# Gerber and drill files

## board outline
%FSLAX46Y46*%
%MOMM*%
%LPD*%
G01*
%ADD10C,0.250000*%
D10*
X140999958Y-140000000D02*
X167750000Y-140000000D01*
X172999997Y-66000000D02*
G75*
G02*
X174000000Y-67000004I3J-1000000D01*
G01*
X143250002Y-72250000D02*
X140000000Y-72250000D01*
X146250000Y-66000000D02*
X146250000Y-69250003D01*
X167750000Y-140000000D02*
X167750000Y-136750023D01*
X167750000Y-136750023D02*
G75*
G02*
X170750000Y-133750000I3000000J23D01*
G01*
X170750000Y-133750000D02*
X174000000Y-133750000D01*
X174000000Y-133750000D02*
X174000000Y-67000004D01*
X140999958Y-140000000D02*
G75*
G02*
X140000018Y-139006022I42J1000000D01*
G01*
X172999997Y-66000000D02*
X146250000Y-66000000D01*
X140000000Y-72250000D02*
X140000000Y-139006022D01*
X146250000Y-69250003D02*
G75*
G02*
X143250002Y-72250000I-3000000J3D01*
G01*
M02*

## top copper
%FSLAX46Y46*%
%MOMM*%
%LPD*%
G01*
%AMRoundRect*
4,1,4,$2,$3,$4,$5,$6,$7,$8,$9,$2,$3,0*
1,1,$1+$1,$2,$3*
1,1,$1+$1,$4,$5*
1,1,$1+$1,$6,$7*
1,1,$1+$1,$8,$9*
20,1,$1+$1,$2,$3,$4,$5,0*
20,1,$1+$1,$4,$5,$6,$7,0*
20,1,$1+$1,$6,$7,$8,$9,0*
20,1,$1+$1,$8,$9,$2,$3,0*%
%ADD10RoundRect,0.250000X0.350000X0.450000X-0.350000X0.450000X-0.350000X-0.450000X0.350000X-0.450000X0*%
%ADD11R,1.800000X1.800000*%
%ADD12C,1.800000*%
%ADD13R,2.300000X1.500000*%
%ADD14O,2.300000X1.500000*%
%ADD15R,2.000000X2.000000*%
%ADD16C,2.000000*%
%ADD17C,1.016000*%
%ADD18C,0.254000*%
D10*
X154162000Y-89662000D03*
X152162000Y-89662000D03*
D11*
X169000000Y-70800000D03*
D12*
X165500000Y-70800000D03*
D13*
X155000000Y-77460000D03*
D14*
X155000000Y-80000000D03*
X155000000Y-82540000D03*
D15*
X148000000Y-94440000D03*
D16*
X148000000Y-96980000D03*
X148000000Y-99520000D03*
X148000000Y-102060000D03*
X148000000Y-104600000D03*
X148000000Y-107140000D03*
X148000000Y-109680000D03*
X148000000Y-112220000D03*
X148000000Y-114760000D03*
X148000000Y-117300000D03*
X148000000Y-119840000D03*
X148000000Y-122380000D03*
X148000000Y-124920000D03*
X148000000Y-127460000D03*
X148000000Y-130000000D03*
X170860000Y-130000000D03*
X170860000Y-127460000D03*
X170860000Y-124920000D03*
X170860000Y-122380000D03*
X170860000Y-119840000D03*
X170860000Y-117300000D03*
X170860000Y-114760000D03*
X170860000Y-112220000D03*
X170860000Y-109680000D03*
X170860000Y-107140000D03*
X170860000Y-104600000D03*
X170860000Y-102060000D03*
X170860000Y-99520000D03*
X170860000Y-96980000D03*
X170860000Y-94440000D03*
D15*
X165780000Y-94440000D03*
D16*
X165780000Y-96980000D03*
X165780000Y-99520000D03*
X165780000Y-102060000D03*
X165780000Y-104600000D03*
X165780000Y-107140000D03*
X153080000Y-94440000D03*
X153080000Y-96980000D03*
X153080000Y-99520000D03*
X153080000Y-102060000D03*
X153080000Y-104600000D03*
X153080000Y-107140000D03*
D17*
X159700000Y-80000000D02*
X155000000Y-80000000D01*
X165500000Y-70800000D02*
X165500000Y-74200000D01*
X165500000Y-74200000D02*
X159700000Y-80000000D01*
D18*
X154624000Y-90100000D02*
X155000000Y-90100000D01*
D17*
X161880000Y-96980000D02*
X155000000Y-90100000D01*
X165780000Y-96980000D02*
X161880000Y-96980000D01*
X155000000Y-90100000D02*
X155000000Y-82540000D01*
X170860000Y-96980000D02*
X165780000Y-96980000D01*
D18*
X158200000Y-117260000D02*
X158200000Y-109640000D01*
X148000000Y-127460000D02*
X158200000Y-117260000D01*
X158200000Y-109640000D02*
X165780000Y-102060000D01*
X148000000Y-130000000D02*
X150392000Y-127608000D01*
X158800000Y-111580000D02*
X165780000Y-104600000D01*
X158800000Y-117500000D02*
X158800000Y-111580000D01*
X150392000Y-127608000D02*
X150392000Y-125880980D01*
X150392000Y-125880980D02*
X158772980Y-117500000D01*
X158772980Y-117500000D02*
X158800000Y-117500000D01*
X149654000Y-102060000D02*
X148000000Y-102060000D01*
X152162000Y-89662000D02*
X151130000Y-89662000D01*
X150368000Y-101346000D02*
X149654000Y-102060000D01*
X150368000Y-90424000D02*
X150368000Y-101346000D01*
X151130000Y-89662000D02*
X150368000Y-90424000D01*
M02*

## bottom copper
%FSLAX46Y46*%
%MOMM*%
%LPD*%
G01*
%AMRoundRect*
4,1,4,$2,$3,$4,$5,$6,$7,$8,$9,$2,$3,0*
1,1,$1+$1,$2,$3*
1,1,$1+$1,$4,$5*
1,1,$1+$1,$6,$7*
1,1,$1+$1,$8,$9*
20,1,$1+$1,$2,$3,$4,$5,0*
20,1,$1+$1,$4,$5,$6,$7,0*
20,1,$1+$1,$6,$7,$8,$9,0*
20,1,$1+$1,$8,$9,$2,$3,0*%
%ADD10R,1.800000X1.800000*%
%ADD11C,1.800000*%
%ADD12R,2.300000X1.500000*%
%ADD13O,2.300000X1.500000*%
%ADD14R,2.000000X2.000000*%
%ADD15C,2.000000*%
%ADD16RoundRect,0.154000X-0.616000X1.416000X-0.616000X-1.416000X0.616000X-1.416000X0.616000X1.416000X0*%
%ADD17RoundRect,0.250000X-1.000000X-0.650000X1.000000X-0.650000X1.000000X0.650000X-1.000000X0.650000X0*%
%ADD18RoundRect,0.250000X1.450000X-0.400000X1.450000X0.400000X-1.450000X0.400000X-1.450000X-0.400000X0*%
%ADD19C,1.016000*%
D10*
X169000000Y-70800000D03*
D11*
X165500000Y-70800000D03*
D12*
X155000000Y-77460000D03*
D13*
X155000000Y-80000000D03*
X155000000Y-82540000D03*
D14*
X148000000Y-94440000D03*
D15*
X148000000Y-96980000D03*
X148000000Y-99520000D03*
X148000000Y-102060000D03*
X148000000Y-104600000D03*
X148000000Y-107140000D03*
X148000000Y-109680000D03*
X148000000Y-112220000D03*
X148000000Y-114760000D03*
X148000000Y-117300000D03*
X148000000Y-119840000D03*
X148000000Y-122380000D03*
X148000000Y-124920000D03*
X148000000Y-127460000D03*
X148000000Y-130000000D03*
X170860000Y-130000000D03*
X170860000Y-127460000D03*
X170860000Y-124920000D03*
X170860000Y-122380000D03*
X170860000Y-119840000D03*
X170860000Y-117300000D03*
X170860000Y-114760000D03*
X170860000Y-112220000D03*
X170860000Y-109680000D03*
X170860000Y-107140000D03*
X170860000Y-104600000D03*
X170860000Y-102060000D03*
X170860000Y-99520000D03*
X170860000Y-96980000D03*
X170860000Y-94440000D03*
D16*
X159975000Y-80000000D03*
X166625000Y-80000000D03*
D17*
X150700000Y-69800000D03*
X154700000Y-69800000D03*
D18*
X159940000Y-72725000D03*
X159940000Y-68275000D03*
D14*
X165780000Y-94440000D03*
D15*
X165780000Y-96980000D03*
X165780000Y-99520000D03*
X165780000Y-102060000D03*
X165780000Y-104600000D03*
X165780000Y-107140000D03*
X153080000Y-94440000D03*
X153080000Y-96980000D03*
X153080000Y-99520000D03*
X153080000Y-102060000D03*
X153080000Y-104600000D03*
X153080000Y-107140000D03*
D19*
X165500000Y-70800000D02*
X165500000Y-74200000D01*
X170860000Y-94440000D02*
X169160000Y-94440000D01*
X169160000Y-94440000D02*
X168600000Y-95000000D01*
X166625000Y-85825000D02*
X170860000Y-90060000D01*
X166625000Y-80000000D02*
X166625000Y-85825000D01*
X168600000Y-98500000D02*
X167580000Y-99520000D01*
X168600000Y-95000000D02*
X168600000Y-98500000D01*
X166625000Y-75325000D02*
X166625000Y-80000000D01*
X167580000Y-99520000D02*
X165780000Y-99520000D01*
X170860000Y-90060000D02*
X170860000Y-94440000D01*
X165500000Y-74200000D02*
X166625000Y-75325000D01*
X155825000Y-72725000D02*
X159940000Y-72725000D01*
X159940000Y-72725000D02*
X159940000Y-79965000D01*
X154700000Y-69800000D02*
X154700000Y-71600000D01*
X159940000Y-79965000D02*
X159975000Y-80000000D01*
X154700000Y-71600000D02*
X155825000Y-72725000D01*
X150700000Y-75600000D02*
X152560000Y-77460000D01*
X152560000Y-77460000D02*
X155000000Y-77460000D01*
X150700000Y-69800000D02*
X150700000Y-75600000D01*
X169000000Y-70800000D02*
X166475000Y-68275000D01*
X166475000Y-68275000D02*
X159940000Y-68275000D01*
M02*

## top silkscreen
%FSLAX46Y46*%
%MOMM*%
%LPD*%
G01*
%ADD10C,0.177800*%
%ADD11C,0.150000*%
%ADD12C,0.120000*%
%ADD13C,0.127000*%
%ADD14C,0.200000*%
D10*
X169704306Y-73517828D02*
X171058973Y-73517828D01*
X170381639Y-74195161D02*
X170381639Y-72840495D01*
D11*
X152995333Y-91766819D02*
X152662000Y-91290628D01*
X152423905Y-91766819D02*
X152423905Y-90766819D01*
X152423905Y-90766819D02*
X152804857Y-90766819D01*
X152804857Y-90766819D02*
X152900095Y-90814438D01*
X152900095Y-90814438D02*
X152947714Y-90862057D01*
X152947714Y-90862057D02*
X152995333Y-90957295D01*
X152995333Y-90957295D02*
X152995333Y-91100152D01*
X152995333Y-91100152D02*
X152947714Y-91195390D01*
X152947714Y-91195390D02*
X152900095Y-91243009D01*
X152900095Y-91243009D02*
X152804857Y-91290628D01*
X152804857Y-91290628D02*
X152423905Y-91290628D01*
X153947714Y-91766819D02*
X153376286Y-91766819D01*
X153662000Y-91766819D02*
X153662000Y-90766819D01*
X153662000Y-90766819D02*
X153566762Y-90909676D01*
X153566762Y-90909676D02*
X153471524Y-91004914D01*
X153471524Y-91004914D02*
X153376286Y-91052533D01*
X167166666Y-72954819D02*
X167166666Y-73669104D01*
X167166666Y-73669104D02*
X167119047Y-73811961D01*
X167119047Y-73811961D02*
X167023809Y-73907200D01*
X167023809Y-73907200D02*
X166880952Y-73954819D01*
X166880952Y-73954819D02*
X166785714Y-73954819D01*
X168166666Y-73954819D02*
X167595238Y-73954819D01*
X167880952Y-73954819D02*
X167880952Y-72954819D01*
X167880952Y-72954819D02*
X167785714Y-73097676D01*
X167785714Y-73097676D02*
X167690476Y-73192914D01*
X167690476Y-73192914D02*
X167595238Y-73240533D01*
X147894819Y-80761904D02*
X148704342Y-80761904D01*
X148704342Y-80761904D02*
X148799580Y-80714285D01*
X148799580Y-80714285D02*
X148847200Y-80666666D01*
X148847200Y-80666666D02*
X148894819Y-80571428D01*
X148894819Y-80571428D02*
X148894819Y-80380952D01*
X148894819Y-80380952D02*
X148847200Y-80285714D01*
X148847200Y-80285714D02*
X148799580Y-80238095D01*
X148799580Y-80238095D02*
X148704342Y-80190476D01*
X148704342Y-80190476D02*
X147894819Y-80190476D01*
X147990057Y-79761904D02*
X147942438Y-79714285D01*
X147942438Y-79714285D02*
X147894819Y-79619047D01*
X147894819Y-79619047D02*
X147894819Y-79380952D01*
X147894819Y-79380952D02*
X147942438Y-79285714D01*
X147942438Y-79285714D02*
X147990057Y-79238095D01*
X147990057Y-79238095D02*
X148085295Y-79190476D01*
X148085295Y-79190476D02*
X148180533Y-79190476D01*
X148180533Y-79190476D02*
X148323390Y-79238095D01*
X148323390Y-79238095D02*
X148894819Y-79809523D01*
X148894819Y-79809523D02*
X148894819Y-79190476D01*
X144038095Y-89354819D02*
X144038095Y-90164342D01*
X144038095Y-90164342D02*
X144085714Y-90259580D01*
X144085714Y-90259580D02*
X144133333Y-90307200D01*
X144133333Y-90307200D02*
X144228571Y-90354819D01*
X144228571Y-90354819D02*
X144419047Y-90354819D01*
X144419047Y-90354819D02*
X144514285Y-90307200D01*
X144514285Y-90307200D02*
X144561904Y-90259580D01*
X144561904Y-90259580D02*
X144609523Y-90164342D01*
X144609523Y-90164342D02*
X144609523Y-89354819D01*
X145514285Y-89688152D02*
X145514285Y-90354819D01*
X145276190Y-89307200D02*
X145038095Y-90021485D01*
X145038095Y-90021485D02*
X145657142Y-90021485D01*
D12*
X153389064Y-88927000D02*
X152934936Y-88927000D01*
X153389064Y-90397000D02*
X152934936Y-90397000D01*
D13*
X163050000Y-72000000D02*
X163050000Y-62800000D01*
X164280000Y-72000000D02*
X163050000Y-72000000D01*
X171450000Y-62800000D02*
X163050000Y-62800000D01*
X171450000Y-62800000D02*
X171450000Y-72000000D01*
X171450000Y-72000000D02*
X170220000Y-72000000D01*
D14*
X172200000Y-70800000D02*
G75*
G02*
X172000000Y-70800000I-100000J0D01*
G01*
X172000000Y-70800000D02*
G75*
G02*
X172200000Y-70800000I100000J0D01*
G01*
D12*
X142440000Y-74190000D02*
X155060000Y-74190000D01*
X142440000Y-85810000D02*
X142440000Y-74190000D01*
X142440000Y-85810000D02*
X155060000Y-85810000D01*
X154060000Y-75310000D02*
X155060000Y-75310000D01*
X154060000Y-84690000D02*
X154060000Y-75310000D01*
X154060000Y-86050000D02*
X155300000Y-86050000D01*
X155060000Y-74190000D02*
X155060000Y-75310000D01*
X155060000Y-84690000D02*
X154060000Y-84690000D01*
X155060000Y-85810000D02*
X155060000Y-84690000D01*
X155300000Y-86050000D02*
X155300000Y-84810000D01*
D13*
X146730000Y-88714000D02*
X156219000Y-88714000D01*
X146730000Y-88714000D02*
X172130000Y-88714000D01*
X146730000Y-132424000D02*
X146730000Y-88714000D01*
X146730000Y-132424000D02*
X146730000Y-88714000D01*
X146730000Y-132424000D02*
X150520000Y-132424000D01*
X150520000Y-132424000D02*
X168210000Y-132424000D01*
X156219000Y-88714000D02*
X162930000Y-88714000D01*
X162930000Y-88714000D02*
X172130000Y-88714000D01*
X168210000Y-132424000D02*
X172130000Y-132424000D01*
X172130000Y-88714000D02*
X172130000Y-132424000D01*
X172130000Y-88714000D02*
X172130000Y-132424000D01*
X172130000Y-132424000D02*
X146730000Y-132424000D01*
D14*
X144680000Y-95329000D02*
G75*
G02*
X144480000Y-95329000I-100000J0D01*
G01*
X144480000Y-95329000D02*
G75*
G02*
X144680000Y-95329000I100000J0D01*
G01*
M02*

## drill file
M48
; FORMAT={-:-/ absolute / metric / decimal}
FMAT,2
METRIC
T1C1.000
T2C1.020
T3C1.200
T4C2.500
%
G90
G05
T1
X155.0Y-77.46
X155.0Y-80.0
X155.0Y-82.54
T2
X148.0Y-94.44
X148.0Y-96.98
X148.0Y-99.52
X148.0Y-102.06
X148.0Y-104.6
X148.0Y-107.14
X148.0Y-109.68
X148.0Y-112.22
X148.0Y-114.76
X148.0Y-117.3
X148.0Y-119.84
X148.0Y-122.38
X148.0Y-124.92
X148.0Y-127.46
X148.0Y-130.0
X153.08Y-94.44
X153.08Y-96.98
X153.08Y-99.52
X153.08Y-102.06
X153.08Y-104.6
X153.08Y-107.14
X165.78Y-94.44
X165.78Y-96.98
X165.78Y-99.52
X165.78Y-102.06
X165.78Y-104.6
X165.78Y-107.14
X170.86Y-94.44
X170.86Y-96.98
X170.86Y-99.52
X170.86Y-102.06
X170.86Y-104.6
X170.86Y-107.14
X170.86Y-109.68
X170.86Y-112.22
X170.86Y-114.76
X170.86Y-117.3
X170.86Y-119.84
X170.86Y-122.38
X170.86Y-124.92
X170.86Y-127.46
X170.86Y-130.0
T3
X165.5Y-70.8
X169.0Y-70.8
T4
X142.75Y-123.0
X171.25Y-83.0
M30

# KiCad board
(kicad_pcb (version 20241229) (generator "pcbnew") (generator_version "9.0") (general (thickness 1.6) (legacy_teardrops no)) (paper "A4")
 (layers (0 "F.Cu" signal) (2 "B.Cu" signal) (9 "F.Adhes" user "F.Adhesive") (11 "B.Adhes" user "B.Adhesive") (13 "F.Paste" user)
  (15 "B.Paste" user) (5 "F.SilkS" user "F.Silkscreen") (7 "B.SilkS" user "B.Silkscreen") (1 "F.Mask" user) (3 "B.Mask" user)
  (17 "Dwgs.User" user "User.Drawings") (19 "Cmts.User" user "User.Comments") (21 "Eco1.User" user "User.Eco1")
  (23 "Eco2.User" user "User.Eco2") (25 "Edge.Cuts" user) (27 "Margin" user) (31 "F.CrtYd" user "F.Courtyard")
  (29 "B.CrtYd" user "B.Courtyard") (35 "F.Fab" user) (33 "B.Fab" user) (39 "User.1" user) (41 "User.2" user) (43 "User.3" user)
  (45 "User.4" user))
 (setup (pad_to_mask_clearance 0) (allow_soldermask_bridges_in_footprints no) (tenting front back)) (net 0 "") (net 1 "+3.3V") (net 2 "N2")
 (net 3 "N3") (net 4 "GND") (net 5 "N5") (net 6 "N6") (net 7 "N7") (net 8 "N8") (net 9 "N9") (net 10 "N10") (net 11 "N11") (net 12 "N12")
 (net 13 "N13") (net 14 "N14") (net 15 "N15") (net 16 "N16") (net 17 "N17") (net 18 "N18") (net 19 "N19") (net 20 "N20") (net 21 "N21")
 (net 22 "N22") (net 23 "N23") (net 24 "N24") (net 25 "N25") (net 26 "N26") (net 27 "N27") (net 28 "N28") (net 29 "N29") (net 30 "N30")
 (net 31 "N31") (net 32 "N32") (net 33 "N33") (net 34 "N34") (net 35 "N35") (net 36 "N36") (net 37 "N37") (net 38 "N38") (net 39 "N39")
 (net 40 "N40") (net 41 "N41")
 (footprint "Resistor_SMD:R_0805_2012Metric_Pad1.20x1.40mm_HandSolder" (layer "F.Cu") (at 153.162 89.662 180)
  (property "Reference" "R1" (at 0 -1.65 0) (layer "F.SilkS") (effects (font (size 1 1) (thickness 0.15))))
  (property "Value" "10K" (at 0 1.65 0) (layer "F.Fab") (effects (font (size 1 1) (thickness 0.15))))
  (fp_line (start -0.227064 0.735) (end 0.227064 0.735) (stroke (width 0.12) (type solid)) (layer "F.SilkS"))
  (fp_line (start -0.227064 -0.735) (end 0.227064 -0.735) (stroke (width 0.12) (type solid)) (layer "F.SilkS"))
  (pad "1" smd roundrect (at -1 0 180) (size 1.2 1.4) (layers "F.Cu" "F.Mask" "F.Paste") (roundrect_rratio 0.208333) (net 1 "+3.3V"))
  (pad "2" smd roundrect (at 1 0 180) (size 1.2 1.4) (layers "F.Cu" "F.Mask" "F.Paste") (roundrect_rratio 0.208333) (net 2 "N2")))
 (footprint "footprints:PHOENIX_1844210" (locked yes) (layer "F.Cu") (at 171.45 62.8 180)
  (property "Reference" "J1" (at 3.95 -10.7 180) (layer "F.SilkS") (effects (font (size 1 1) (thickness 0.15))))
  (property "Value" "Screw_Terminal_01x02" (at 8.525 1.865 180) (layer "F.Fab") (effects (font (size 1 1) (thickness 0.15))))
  (fp_line (start 8.4 -9.2) (end 8.4 0) (stroke (width 0.127) (type solid)) (layer "F.SilkS"))
  (fp_line (start 7.17 -9.2) (end 8.4 -9.2) (stroke (width 0.127) (type solid)) (layer "F.SilkS"))
  (fp_line (start 0 0) (end 8.4 0) (stroke (width 0.127) (type solid)) (layer "F.SilkS"))
  (fp_line (start 0 0) (end 0 -9.2) (stroke (width 0.127) (type solid)) (layer "F.SilkS"))
  (fp_line (start 0 -9.2) (end 1.23 -9.2) (stroke (width 0.127) (type solid)) (layer "F.SilkS"))
  (fp_circle (center -0.65 -8) (end -0.55 -8) (stroke (width 0.2) (type solid)) (fill no) (layer "F.SilkS"))
  (pad "01" thru_hole rect (at 2.45 -8 180) (size 1.8 1.8) (drill 1.2) (layers "*.Cu" "*.Mask") (remove_unused_layers no) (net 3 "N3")
   (solder_mask_margin 0.102))
  (pad "02" thru_hole circle (at 5.95 -8 180) (size 1.8 1.8) (drill 1.2) (layers "*.Cu" "*.Mask") (remove_unused_layers no) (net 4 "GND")
   (solder_mask_margin 0.102)))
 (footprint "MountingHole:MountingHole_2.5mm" (layer "F.Cu") (at 171.25 83)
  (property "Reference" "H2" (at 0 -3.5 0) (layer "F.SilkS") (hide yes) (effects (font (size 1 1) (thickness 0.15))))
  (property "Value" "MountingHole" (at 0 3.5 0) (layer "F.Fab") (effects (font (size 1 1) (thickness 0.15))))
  (pad "" np_thru_hole circle (at 0 0) (size 2.5 2.5) (drill 2.5) (layers "*.Cu" "*.Mask")))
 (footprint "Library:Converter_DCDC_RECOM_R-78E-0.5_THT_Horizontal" (layer "F.Cu") (at 155 82.54 90)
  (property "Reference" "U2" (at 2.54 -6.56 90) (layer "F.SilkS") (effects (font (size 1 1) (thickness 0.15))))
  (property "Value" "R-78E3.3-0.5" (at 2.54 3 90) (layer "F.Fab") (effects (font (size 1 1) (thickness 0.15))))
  (fp_line (start 8.35 -12.56) (end 8.35 0.06) (stroke (width 0.12) (type solid)) (layer "F.SilkS"))
  (fp_line (start -3.27 -12.56) (end 8.35 -12.56) (stroke (width 0.12) (type solid)) (layer "F.SilkS"))
  (fp_line (start -3.27 -12.56) (end -3.27 0.06) (stroke (width 0.12) (type solid)) (layer "F.SilkS"))
  (fp_line (start 7.23 -0.94) (end 7.23 0.06) (stroke (width 0.12) (type solid)) (layer "F.SilkS"))
  (fp_line (start -2.15 -0.94) (end 7.23 -0.94) (stroke (width 0.12) (type solid)) (layer "F.SilkS"))
  (fp_line (start -3.51 -0.94) (end -3.51 0.3) (stroke (width 0.12) (type solid)) (layer "F.SilkS"))
  (fp_line (start 8.35 0.06) (end 7.23 0.06) (stroke (width 0.12) (type solid)) (layer "F.SilkS"))
  (fp_line (start -2.15 0.06) (end -2.15 -0.94) (stroke (width 0.12) (type solid)) (layer "F.SilkS"))
  (fp_line (start -3.27 0.06) (end -2.15 0.06) (stroke (width 0.12) (type solid)) (layer "F.SilkS"))
  (fp_line (start -3.51 0.3) (end -2.27 0.3) (stroke (width 0.12) (type solid)) (layer "F.SilkS"))
  (pad "1" thru_hole rect (at 5.08 0 90) (size 1.5 2.3) (drill 1) (layers "*.Cu" "*.Mask") (remove_unused_layers no) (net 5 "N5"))
  (pad "2" thru_hole oval (at 2.54 0 90) (size 1.5 2.3) (drill 1) (layers "*.Cu" "*.Mask") (remove_unused_layers no) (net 4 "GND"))
  (pad "3" thru_hole oval (at 0 0 90) (size 1.5 2.3) (drill 1) (layers "*.Cu" "*.Mask") (remove_unused_layers no) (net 1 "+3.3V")))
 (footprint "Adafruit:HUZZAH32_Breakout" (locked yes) (layer "F.Cu") (at 159.43 110.569)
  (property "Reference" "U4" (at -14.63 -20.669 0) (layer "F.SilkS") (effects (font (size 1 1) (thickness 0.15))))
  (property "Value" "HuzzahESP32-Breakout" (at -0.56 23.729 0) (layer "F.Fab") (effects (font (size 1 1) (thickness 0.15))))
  (fp_line (start -12.7 -21.855) (end -3.211 -21.855) (stroke (width 0.127) (type solid)) (layer "F.SilkS"))
  (fp_line (start -12.7 -21.855) (end 12.7 -21.855) (stroke (width 0.127) (type solid)) (layer "F.SilkS"))
  (fp_line (start -12.7 21.855) (end -12.7 -21.855) (stroke (width 0.127) (type solid)) (layer "F.SilkS"))
  (fp_line (start -12.7 21.855) (end -12.7 -21.855) (stroke (width 0.127) (type solid)) (layer "F.SilkS"))
  (fp_line (start -12.7 21.855) (end -8.91 21.855) (stroke (width 0.127) (type solid)) (layer "F.SilkS"))
  (fp_line (start -8.91 21.855) (end 8.78 21.855) (stroke (width 0.127) (type solid)) (layer "F.SilkS"))
  (fp_line (start -3.211 -21.855) (end 3.5 -21.855) (stroke (width 0.127) (type solid)) (layer "F.SilkS"))
  (fp_line (start 3.5 -21.855) (end 12.7 -21.855) (stroke (width 0.127) (type solid)) (layer "F.SilkS"))
  (fp_line (start 8.78 21.855) (end 12.7 21.855) (stroke (width 0.127) (type solid)) (layer "F.SilkS"))
  (fp_line (start 12.7 -21.855) (end 12.7 21.855) (stroke (width 0.127) (type solid)) (layer "F.SilkS"))
  (fp_line (start 12.7 -21.855) (end 12.7 21.855) (stroke (width 0.127) (type solid)) (layer "F.SilkS"))
  (fp_line (start 12.7 21.855) (end -12.7 21.855) (stroke (width 0.127) (type solid)) (layer "F.SilkS"))
  (fp_circle (center -14.85 -15.24) (end -14.75 -15.24) (stroke (width 0.2) (type solid)) (fill no) (layer "F.SilkS"))
  (pad "1" thru_hole rect (at -11.43 -16.129) (size 2 2) (drill 1.02) (layers "*.Cu" "*.Mask") (remove_unused_layers no) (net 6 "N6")
   (solder_mask_margin 0.102))
  (pad "2" thru_hole circle (at -11.43 -13.589) (size 2 2) (drill 1.02) (layers "*.Cu" "*.Mask") (remove_unused_layers no) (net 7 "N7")
   (solder_mask_margin 0.102))
  (pad "3" thru_hole circle (at -11.43 -11.049) (size 2 2) (drill 1.02) (layers "*.Cu" "*.Mask") (remove_unused_layers no) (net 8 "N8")
   (solder_mask_margin 0.102))
  (pad "4" thru_hole circle (at -11.43 -8.509) (size 2 2) (drill 1.02) (layers "*.Cu" "*.Mask") (remove_unused_layers no) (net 2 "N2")
   (solder_mask_margin 0.102))
  (pad "5" thru_hole circle (at -11.43 -5.969) (size 2 2) (drill 1.02) (layers "*.Cu" "*.Mask") (remove_unused_layers no) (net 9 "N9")
   (solder_mask_margin 0.102))
  (pad "6" thru_hole circle (at -11.43 -3.429) (size 2 2) (drill 1.02) (layers "*.Cu" "*.Mask") (remove_unused_layers no) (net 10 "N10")
   (solder_mask_margin 0.102))
  (pad "7" thru_hole circle (at -11.43 -0.889) (size 2 2) (drill 1.02) (layers "*.Cu" "*.Mask") (remove_unused_layers no) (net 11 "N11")
   (solder_mask_margin 0.102))
  (pad "8" thru_hole circle (at -11.43 1.651) (size 2 2) (drill 1.02) (layers "*.Cu" "*.Mask") (remove_unused_layers no) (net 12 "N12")
   (solder_mask_margin 0.102))
  (pad "9" thru_hole circle (at -11.43 4.191) (size 2 2) (drill 1.02) (layers "*.Cu" "*.Mask") (remove_unused_layers no) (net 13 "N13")
   (solder_mask_margin 0.102))
  (pad "10" thru_hole circle (at -11.43 6.731) (size 2 2) (drill 1.02) (layers "*.Cu" "*.Mask") (remove_unused_layers no) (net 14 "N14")
   (solder_mask_margin 0.102))
  (pad "11" thru_hole circle (at -11.43 9.271) (size 2 2) (drill 1.02) (layers "*.Cu" "*.Mask") (remove_unused_layers no) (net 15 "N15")
   (solder_mask_margin 0.102))
  (pad "12" thru_hole circle (at -11.43 11.811) (size 2 2) (drill 1.02) (layers "*.Cu" "*.Mask") (remove_unused_layers no) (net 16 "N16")
   (solder_mask_margin 0.102))
  (pad "13" thru_hole circle (at -11.43 14.351) (size 2 2) (drill 1.02) (layers "*.Cu" "*.Mask") (remove_unused_layers no) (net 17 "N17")
   (solder_mask_margin 0.102))
  (pad "14" thru_hole circle (at -11.43 16.891) (size 2 2) (drill 1.02) (layers "*.Cu" "*.Mask") (remove_unused_layers no) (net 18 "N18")
   (solder_mask_margin 0.102))
  (pad "15" thru_hole circle (at -11.43 19.431) (size 2 2) (drill 1.02) (layers "*.Cu" "*.Mask") (remove_unused_layers no) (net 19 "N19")
   (solder_mask_margin 0.102))
  (pad "16" thru_hole circle (at 11.43 19.431) (size 2 2) (drill 1.02) (layers "*.Cu" "*.Mask") (remove_unused_layers no) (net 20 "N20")
   (solder_mask_margin 0.102))
  (pad "17" thru_hole circle (at 11.43 16.891) (size 2 2) (drill 1.02) (layers "*.Cu" "*.Mask") (remove_unused_layers no) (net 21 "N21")
   (solder_mask_margin 0.102))
  (pad "18" thru_hole circle (at 11.43 14.351) (size 2 2) (drill 1.02) (layers "*.Cu" "*.Mask") (remove_unused_layers no) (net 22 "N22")
   (solder_mask_margin 0.102))
  (pad "19" thru_hole circle (at 11.43 11.811) (size 2 2) (drill 1.02) (layers "*.Cu" "*.Mask") (remove_unused_layers no) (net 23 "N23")
   (solder_mask_margin 0.102))
  (pad "20" thru_hole circle (at 11.43 9.271) (size 2 2) (drill 1.02) (layers "*.Cu" "*.Mask") (remove_unused_layers no) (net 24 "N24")
   (solder_mask_margin 0.102))
  (pad "21" thru_hole circle (at 11.43 6.731) (size 2 2) (drill 1.02) (layers "*.Cu" "*.Mask") (remove_unused_layers no) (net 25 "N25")
   (solder_mask_margin 0.102))
  (pad "22" thru_hole circle (at 11.43 4.191) (size 2 2) (drill 1.02) (layers "*.Cu" "*.Mask") (remove_unused_layers no) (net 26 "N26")
   (solder_mask_margin 0.102))
  (pad "23" thru_hole circle (at 11.43 1.651) (size 2 2) (drill 1.02) (layers "*.Cu" "*.Mask") (remove_unused_layers no) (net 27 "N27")
   (solder_mask_margin 0.102))
  (pad "24" thru_hole circle (at 11.43 -0.889) (size 2 2) (drill 1.02) (layers "*.Cu" "*.Mask") (remove_unused_layers no) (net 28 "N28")
   (solder_mask_margin 0.102))
  (pad "25" thru_hole circle (at 11.43 -3.429) (size 2 2) (drill 1.02) (layers "*.Cu" "*.Mask") (remove_unused_layers no) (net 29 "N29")
   (solder_mask_margin 0.102))
  (pad "26" thru_hole circle (at 11.43 -5.969) (size 2 2) (drill 1.02) (layers "*.Cu" "*.Mask") (remove_unused_layers no) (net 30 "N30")
   (solder_mask_margin 0.102))
  (pad "27" thru_hole circle (at 11.43 -8.509) (size 2 2) (drill 1.02) (layers "*.Cu" "*.Mask") (remove_unused_layers no) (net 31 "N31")
   (solder_mask_margin 0.102))
  (pad "28" thru_hole circle (at 11.43 -11.049) (size 2 2) (drill 1.02) (layers "*.Cu" "*.Mask") (remove_unused_layers no) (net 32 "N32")
   (solder_mask_margin 0.102))
  (pad "29" thru_hole circle (at 11.43 -13.589) (size 2 2) (drill 1.02) (layers "*.Cu" "*.Mask") (remove_unused_layers no) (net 1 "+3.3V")
   (solder_mask_margin 0.102))
  (pad "30" thru_hole circle (at 11.43 -16.129) (size 2 2) (drill 1.02) (layers "*.Cu" "*.Mask") (remove_unused_layers no) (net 4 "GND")
   (solder_mask_margin 0.102))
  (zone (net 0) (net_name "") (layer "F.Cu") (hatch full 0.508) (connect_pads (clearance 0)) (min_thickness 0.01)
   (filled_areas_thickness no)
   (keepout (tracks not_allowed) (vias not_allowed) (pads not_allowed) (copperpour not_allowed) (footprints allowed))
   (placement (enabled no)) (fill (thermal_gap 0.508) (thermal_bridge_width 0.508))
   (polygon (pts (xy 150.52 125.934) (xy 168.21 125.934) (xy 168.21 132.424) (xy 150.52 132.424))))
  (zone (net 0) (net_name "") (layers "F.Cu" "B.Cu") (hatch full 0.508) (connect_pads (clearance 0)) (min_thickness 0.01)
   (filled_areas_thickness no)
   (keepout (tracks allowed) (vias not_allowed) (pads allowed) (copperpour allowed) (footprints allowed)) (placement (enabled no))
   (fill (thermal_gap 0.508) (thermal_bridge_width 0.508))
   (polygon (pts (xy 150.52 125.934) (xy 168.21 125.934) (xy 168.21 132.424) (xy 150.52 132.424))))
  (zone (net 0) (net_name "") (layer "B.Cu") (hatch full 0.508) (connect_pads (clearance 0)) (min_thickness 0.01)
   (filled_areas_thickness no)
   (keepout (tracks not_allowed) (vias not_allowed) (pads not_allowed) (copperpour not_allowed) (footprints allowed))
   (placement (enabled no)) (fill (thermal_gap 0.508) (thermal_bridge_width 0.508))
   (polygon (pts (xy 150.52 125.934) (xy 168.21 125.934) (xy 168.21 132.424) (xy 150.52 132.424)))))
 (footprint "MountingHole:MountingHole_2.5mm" (layer "F.Cu") (at 142.75 123)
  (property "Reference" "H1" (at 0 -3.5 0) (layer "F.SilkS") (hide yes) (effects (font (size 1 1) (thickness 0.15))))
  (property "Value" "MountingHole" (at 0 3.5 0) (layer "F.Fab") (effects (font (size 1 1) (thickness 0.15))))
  (pad "" np_thru_hole circle (at 0 0) (size 2.5 2.5) (drill 2.5) (layers "*.Cu" "*.Mask")))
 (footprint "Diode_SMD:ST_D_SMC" (layer "B.Cu") (at 163.3 80)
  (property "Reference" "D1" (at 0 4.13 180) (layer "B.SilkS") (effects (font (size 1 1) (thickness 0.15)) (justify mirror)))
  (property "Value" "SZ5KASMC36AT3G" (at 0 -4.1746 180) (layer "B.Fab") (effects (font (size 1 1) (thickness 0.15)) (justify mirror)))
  (pad "1" smd roundrect (at -3.325 0 270) (size 3.14 1.54) (layers "B.Cu" "B.Mask" "B.Paste") (roundrect_rratio 0.1) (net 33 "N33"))
  (pad "2" smd roundrect (at 3.325 0 270) (size 3.14 1.54) (layers "B.Cu" "B.Mask" "B.Paste") (roundrect_rratio 0.1) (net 4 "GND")))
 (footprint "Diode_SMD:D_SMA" (layer "B.Cu") (at 152.7 69.8)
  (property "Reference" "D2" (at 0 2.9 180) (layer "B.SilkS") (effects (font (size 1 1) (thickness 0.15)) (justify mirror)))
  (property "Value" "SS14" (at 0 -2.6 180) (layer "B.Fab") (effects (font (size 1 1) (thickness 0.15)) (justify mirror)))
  (pad "1" smd roundrect (at -2 0) (size 2.5 1.8) (layers "B.Cu" "B.Mask" "B.Paste") (roundrect_rratio 0.1388888889) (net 5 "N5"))
  (pad "2" smd roundrect (at 2 0) (size 2.5 1.8) (layers "B.Cu" "B.Mask" "B.Paste") (roundrect_rratio 0.1388888889) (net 33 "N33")))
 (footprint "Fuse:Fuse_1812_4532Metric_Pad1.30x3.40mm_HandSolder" (layer "B.Cu") (at 159.94 70.5 90)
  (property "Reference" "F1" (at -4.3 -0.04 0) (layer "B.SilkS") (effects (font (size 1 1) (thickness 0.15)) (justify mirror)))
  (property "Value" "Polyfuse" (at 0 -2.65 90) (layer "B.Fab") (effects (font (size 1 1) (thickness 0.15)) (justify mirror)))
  (pad "1" smd roundrect (at -2.225 0 90) (size 1.3 3.4) (layers "B.Cu" "B.Mask" "B.Paste") (roundrect_rratio 0.192308) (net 33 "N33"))
  (pad "2" smd roundrect (at 2.225 0 90) (size 1.3 3.4) (layers "B.Cu" "B.Mask" "B.Paste") (roundrect_rratio 0.192308) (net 3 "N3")))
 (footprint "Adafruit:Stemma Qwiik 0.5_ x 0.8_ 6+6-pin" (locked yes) (layer "B.Cu") (at 159.43 100.79 180)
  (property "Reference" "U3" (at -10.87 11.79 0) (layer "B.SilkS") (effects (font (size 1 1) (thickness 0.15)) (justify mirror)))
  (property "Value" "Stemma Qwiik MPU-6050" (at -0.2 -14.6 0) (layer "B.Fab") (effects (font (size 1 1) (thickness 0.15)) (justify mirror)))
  (pad "1" thru_hole rect (at -6.35 6.35 180) (size 2 2) (drill 1.02) (layers "*.Cu" "*.Mask") (remove_unused_layers no) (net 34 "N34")
   (solder_mask_margin 0.102))
  (pad "2" thru_hole circle (at -6.35 3.81 180) (size 2 2) (drill 1.02) (layers "*.Cu" "*.Mask") (remove_unused_layers no) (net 1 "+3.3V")
   (solder_mask_margin 0.102))
  (pad "3" thru_hole circle (at -6.35 1.27 180) (size 2 2) (drill 1.02) (layers "*.Cu" "*.Mask") (remove_unused_layers no) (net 4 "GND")
   (solder_mask_margin 0.102))
  (pad "4" thru_hole circle (at -6.35 -1.27 180) (size 2 2) (drill 1.02) (layers "*.Cu" "*.Mask") (remove_unused_layers no) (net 18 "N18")
   (solder_mask_margin 0.102))
  (pad "5" thru_hole circle (at -6.35 -3.81 180) (size 2 2) (drill 1.02) (layers "*.Cu" "*.Mask") (remove_unused_layers no) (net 19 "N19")
   (solder_mask_margin 0.102))
  (pad "6" thru_hole circle (at -6.35 -6.35 180) (size 2 2) (drill 1.02) (layers "*.Cu" "*.Mask") (remove_unused_layers no) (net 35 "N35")
   (solder_mask_margin 0.102))
  (pad "7" thru_hole circle (at 6.35 6.35 180) (size 2 2) (drill 1.02) (layers "*.Cu" "*.Mask") (remove_unused_layers no) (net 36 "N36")
   (solder_mask_margin 0.102))
  (pad "8" thru_hole circle (at 6.35 3.81 180) (size 2 2) (drill 1.02) (layers "*.Cu" "*.Mask") (remove_unused_layers no) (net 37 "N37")
   (solder_mask_margin 0.102))
  (pad "9" thru_hole circle (at 6.35 1.27 180) (size 2 2) (drill 1.02) (layers "*.Cu" "*.Mask") (remove_unused_layers no) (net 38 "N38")
   (solder_mask_margin 0.102))
  (pad "10" thru_hole circle (at 6.35 -1.27 180) (size 2 2) (drill 1.02) (layers "*.Cu" "*.Mask") (remove_unused_layers no) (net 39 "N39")
   (solder_mask_margin 0.102))
  (pad "11" thru_hole circle (at 6.35 -3.81 180) (size 2 2) (drill 1.02) (layers "*.Cu" "*.Mask") (remove_unused_layers no) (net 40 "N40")
   (solder_mask_margin 0.102))
  (pad "12" thru_hole circle (at 6.35 -6.35 180) (size 2 2) (drill 1.02) (layers "*.Cu" "*.Mask") (remove_unused_layers no) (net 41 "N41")
   (solder_mask_margin 0.102)))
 (gr_line (start 140.999958 140) (end 167.75 140) (stroke (width 0.25) (type default)) (layer "Edge.Cuts"))
 (gr_arc (start 172.999997 66) (mid 173.707107 66.292894) (end 174 67.000004) (stroke (width 0.25) (type default)) (layer "Edge.Cuts"))
 (gr_line (start 143.250002 72.25) (end 140 72.25) (stroke (width 0.25) (type default)) (layer "Edge.Cuts"))
 (gr_line (start 146.25 66) (end 146.25 69.250003) (stroke (width 0.25) (type default)) (layer "Edge.Cuts"))
 (gr_line (start 167.75 140) (end 167.75 136.750023) (stroke (width 0.25) (type default)) (layer "Edge.Cuts"))
 (gr_arc (start 167.75 136.750023) (mid 168.628672 134.628688) (end 170.75 133.75) (stroke (width 0.25) (type default)) (layer "Edge.Cuts"))
 (gr_line (start 170.75 133.75) (end 174 133.75) (stroke (width 0.25) (type default)) (layer "Edge.Cuts"))
 (gr_line (start 174 133.75) (end 174 67.000004) (stroke (width 0.25) (type default)) (layer "Edge.Cuts"))
 (gr_arc (start 140.999958 140) (mid 140.295011 139.709218) (end 140 139.006022) (stroke (width 0.25) (type default)) (layer "Edge.Cuts"))
 (gr_line (start 172.999997 66) (end 146.25 66) (stroke (width 0.25) (type solid)) (layer "Edge.Cuts"))
 (gr_line (start 140 72.25) (end 140 139.006022) (stroke (width 0.25) (type default)) (layer "Edge.Cuts"))
 (gr_arc (start 146.25 69.250003) (mid 145.37132 71.371321) (end 143.250002 72.25) (stroke (width 0.25) (type default)) (layer "Edge.Cuts"))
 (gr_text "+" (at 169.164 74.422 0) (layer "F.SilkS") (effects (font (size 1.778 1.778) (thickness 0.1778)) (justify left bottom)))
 (segment (start 159.7 80) (end 155 80) (width 1.016) (layer "F.Cu") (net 4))
 (segment (start 165.5 70.8) (end 165.5 74.2) (width 1.016) (layer "F.Cu") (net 4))
 (segment (start 165.5 74.2) (end 159.7 80) (width 1.016) (layer "F.Cu") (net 4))
 (segment (start 165.5 70.8) (end 165.5 74.2) (width 1.016) (layer "B.Cu") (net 4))
 (segment (start 170.86 94.44) (end 169.16 94.44) (width 1.016) (layer "B.Cu") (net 4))
 (segment (start 169.16 94.44) (end 168.6 95) (width 1.016) (layer "B.Cu") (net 4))
 (segment (start 166.625 85.825) (end 170.86 90.06) (width 1.016) (layer "B.Cu") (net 4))
 (segment (start 166.625 80) (end 166.625 85.825) (width 1.016) (layer "B.Cu") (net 4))
 (segment (start 168.6 98.5) (end 167.58 99.52) (width 1.016) (layer "B.Cu") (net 4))
 (segment (start 168.6 95) (end 168.6 98.5) (width 1.016) (layer "B.Cu") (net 4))
 (segment (start 166.625 75.325) (end 166.625 80) (width 1.016) (layer "B.Cu") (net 4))
 (segment (start 167.58 99.52) (end 165.78 99.52) (width 1.016) (layer "B.Cu") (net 4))
 (segment (start 170.86 90.06) (end 170.86 94.44) (width 1.016) (layer "B.Cu") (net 4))
 (segment (start 165.5 74.2) (end 166.625 75.325) (width 1.016) (layer "B.Cu") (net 4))
 (segment (start 155.825 72.725) (end 159.94 72.725) (width 1.016) (layer "B.Cu") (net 33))
 (segment (start 159.94 72.725) (end 159.94 79.965) (width 1.016) (layer "B.Cu") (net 33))
 (segment (start 154.7 69.8) (end 154.7 71.6) (width 1.016) (layer "B.Cu") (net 33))
 (segment (start 159.94 79.965) (end 159.975 80) (width 1.016) (layer "B.Cu") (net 33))
 (segment (start 154.7 71.6) (end 155.825 72.725) (width 1.016) (layer "B.Cu") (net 33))
 (segment (start 154.624 90.1) (end 155 90.1) (width 0.254) (layer "F.Cu") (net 1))
 (segment (start 161.88 96.98) (end 155 90.1) (width 1.016) (layer "F.Cu") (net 1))
 (segment (start 165.78 96.98) (end 161.88 96.98) (width 1.016) (layer "F.Cu") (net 1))
 (segment (start 155 90.1) (end 155 82.54) (width 1.016) (layer "F.Cu") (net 1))
 (segment (start 170.86 96.98) (end 165.78 96.98) (width 1.016) (layer "F.Cu") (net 1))
 (segment (start 150.7 75.6) (end 152.56 77.46) (width 1.016) (layer "B.Cu") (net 5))
 (segment (start 152.56 77.46) (end 155 77.46) (width 1.016) (layer "B.Cu") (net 5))
 (segment (start 150.7 69.8) (end 150.7 75.6) (width 1.016) (layer "B.Cu") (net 5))
 (segment (start 158.2 117.26) (end 158.2 109.64) (width 0.254) (layer "F.Cu") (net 18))
 (segment (start 148 127.46) (end 158.2 117.26) (width 0.254) (layer "F.Cu") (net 18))
 (segment (start 158.2 109.64) (end 165.78 102.06) (width 0.254) (layer "F.Cu") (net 18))
 (segment (start 148 130) (end 150.392 127.608) (width 0.254) (layer "F.Cu") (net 19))
 (segment (start 158.8 111.58) (end 165.78 104.6) (width 0.254) (layer "F.Cu") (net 19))
 (segment (start 158.8 117.5) (end 158.8 111.58) (width 0.254) (layer "F.Cu") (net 19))
 (segment (start 150.392 127.608) (end 150.392 125.88098) (width 0.254) (layer "F.Cu") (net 19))
 (segment (start 150.392 125.88098) (end 158.77298 117.5) (width 0.254) (layer "F.Cu") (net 19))
 (segment (start 158.77298 117.5) (end 158.8 117.5) (width 0.254) (layer "F.Cu") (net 19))
 (segment (start 169 70.8) (end 166.475 68.275) (width 1.016) (layer "B.Cu") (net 3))
 (segment (start 166.475 68.275) (end 159.94 68.275) (width 1.016) (layer "B.Cu") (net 3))
 (segment (start 149.654 102.06) (end 148 102.06) (width 0.254) (layer "F.Cu") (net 2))
 (segment (start 152.162 89.662) (end 151.13 89.662) (width 0.254) (layer "F.Cu") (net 2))
 (segment (start 150.368 101.346) (end 149.654 102.06) (width 0.254) (layer "F.Cu") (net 2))
 (segment (start 150.368 90.424) (end 150.368 101.346) (width 0.254) (layer "F.Cu") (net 2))
 (segment (start 151.13 89.662) (end 150.368 90.424) (width 0.254) (layer "F.Cu") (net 2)))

